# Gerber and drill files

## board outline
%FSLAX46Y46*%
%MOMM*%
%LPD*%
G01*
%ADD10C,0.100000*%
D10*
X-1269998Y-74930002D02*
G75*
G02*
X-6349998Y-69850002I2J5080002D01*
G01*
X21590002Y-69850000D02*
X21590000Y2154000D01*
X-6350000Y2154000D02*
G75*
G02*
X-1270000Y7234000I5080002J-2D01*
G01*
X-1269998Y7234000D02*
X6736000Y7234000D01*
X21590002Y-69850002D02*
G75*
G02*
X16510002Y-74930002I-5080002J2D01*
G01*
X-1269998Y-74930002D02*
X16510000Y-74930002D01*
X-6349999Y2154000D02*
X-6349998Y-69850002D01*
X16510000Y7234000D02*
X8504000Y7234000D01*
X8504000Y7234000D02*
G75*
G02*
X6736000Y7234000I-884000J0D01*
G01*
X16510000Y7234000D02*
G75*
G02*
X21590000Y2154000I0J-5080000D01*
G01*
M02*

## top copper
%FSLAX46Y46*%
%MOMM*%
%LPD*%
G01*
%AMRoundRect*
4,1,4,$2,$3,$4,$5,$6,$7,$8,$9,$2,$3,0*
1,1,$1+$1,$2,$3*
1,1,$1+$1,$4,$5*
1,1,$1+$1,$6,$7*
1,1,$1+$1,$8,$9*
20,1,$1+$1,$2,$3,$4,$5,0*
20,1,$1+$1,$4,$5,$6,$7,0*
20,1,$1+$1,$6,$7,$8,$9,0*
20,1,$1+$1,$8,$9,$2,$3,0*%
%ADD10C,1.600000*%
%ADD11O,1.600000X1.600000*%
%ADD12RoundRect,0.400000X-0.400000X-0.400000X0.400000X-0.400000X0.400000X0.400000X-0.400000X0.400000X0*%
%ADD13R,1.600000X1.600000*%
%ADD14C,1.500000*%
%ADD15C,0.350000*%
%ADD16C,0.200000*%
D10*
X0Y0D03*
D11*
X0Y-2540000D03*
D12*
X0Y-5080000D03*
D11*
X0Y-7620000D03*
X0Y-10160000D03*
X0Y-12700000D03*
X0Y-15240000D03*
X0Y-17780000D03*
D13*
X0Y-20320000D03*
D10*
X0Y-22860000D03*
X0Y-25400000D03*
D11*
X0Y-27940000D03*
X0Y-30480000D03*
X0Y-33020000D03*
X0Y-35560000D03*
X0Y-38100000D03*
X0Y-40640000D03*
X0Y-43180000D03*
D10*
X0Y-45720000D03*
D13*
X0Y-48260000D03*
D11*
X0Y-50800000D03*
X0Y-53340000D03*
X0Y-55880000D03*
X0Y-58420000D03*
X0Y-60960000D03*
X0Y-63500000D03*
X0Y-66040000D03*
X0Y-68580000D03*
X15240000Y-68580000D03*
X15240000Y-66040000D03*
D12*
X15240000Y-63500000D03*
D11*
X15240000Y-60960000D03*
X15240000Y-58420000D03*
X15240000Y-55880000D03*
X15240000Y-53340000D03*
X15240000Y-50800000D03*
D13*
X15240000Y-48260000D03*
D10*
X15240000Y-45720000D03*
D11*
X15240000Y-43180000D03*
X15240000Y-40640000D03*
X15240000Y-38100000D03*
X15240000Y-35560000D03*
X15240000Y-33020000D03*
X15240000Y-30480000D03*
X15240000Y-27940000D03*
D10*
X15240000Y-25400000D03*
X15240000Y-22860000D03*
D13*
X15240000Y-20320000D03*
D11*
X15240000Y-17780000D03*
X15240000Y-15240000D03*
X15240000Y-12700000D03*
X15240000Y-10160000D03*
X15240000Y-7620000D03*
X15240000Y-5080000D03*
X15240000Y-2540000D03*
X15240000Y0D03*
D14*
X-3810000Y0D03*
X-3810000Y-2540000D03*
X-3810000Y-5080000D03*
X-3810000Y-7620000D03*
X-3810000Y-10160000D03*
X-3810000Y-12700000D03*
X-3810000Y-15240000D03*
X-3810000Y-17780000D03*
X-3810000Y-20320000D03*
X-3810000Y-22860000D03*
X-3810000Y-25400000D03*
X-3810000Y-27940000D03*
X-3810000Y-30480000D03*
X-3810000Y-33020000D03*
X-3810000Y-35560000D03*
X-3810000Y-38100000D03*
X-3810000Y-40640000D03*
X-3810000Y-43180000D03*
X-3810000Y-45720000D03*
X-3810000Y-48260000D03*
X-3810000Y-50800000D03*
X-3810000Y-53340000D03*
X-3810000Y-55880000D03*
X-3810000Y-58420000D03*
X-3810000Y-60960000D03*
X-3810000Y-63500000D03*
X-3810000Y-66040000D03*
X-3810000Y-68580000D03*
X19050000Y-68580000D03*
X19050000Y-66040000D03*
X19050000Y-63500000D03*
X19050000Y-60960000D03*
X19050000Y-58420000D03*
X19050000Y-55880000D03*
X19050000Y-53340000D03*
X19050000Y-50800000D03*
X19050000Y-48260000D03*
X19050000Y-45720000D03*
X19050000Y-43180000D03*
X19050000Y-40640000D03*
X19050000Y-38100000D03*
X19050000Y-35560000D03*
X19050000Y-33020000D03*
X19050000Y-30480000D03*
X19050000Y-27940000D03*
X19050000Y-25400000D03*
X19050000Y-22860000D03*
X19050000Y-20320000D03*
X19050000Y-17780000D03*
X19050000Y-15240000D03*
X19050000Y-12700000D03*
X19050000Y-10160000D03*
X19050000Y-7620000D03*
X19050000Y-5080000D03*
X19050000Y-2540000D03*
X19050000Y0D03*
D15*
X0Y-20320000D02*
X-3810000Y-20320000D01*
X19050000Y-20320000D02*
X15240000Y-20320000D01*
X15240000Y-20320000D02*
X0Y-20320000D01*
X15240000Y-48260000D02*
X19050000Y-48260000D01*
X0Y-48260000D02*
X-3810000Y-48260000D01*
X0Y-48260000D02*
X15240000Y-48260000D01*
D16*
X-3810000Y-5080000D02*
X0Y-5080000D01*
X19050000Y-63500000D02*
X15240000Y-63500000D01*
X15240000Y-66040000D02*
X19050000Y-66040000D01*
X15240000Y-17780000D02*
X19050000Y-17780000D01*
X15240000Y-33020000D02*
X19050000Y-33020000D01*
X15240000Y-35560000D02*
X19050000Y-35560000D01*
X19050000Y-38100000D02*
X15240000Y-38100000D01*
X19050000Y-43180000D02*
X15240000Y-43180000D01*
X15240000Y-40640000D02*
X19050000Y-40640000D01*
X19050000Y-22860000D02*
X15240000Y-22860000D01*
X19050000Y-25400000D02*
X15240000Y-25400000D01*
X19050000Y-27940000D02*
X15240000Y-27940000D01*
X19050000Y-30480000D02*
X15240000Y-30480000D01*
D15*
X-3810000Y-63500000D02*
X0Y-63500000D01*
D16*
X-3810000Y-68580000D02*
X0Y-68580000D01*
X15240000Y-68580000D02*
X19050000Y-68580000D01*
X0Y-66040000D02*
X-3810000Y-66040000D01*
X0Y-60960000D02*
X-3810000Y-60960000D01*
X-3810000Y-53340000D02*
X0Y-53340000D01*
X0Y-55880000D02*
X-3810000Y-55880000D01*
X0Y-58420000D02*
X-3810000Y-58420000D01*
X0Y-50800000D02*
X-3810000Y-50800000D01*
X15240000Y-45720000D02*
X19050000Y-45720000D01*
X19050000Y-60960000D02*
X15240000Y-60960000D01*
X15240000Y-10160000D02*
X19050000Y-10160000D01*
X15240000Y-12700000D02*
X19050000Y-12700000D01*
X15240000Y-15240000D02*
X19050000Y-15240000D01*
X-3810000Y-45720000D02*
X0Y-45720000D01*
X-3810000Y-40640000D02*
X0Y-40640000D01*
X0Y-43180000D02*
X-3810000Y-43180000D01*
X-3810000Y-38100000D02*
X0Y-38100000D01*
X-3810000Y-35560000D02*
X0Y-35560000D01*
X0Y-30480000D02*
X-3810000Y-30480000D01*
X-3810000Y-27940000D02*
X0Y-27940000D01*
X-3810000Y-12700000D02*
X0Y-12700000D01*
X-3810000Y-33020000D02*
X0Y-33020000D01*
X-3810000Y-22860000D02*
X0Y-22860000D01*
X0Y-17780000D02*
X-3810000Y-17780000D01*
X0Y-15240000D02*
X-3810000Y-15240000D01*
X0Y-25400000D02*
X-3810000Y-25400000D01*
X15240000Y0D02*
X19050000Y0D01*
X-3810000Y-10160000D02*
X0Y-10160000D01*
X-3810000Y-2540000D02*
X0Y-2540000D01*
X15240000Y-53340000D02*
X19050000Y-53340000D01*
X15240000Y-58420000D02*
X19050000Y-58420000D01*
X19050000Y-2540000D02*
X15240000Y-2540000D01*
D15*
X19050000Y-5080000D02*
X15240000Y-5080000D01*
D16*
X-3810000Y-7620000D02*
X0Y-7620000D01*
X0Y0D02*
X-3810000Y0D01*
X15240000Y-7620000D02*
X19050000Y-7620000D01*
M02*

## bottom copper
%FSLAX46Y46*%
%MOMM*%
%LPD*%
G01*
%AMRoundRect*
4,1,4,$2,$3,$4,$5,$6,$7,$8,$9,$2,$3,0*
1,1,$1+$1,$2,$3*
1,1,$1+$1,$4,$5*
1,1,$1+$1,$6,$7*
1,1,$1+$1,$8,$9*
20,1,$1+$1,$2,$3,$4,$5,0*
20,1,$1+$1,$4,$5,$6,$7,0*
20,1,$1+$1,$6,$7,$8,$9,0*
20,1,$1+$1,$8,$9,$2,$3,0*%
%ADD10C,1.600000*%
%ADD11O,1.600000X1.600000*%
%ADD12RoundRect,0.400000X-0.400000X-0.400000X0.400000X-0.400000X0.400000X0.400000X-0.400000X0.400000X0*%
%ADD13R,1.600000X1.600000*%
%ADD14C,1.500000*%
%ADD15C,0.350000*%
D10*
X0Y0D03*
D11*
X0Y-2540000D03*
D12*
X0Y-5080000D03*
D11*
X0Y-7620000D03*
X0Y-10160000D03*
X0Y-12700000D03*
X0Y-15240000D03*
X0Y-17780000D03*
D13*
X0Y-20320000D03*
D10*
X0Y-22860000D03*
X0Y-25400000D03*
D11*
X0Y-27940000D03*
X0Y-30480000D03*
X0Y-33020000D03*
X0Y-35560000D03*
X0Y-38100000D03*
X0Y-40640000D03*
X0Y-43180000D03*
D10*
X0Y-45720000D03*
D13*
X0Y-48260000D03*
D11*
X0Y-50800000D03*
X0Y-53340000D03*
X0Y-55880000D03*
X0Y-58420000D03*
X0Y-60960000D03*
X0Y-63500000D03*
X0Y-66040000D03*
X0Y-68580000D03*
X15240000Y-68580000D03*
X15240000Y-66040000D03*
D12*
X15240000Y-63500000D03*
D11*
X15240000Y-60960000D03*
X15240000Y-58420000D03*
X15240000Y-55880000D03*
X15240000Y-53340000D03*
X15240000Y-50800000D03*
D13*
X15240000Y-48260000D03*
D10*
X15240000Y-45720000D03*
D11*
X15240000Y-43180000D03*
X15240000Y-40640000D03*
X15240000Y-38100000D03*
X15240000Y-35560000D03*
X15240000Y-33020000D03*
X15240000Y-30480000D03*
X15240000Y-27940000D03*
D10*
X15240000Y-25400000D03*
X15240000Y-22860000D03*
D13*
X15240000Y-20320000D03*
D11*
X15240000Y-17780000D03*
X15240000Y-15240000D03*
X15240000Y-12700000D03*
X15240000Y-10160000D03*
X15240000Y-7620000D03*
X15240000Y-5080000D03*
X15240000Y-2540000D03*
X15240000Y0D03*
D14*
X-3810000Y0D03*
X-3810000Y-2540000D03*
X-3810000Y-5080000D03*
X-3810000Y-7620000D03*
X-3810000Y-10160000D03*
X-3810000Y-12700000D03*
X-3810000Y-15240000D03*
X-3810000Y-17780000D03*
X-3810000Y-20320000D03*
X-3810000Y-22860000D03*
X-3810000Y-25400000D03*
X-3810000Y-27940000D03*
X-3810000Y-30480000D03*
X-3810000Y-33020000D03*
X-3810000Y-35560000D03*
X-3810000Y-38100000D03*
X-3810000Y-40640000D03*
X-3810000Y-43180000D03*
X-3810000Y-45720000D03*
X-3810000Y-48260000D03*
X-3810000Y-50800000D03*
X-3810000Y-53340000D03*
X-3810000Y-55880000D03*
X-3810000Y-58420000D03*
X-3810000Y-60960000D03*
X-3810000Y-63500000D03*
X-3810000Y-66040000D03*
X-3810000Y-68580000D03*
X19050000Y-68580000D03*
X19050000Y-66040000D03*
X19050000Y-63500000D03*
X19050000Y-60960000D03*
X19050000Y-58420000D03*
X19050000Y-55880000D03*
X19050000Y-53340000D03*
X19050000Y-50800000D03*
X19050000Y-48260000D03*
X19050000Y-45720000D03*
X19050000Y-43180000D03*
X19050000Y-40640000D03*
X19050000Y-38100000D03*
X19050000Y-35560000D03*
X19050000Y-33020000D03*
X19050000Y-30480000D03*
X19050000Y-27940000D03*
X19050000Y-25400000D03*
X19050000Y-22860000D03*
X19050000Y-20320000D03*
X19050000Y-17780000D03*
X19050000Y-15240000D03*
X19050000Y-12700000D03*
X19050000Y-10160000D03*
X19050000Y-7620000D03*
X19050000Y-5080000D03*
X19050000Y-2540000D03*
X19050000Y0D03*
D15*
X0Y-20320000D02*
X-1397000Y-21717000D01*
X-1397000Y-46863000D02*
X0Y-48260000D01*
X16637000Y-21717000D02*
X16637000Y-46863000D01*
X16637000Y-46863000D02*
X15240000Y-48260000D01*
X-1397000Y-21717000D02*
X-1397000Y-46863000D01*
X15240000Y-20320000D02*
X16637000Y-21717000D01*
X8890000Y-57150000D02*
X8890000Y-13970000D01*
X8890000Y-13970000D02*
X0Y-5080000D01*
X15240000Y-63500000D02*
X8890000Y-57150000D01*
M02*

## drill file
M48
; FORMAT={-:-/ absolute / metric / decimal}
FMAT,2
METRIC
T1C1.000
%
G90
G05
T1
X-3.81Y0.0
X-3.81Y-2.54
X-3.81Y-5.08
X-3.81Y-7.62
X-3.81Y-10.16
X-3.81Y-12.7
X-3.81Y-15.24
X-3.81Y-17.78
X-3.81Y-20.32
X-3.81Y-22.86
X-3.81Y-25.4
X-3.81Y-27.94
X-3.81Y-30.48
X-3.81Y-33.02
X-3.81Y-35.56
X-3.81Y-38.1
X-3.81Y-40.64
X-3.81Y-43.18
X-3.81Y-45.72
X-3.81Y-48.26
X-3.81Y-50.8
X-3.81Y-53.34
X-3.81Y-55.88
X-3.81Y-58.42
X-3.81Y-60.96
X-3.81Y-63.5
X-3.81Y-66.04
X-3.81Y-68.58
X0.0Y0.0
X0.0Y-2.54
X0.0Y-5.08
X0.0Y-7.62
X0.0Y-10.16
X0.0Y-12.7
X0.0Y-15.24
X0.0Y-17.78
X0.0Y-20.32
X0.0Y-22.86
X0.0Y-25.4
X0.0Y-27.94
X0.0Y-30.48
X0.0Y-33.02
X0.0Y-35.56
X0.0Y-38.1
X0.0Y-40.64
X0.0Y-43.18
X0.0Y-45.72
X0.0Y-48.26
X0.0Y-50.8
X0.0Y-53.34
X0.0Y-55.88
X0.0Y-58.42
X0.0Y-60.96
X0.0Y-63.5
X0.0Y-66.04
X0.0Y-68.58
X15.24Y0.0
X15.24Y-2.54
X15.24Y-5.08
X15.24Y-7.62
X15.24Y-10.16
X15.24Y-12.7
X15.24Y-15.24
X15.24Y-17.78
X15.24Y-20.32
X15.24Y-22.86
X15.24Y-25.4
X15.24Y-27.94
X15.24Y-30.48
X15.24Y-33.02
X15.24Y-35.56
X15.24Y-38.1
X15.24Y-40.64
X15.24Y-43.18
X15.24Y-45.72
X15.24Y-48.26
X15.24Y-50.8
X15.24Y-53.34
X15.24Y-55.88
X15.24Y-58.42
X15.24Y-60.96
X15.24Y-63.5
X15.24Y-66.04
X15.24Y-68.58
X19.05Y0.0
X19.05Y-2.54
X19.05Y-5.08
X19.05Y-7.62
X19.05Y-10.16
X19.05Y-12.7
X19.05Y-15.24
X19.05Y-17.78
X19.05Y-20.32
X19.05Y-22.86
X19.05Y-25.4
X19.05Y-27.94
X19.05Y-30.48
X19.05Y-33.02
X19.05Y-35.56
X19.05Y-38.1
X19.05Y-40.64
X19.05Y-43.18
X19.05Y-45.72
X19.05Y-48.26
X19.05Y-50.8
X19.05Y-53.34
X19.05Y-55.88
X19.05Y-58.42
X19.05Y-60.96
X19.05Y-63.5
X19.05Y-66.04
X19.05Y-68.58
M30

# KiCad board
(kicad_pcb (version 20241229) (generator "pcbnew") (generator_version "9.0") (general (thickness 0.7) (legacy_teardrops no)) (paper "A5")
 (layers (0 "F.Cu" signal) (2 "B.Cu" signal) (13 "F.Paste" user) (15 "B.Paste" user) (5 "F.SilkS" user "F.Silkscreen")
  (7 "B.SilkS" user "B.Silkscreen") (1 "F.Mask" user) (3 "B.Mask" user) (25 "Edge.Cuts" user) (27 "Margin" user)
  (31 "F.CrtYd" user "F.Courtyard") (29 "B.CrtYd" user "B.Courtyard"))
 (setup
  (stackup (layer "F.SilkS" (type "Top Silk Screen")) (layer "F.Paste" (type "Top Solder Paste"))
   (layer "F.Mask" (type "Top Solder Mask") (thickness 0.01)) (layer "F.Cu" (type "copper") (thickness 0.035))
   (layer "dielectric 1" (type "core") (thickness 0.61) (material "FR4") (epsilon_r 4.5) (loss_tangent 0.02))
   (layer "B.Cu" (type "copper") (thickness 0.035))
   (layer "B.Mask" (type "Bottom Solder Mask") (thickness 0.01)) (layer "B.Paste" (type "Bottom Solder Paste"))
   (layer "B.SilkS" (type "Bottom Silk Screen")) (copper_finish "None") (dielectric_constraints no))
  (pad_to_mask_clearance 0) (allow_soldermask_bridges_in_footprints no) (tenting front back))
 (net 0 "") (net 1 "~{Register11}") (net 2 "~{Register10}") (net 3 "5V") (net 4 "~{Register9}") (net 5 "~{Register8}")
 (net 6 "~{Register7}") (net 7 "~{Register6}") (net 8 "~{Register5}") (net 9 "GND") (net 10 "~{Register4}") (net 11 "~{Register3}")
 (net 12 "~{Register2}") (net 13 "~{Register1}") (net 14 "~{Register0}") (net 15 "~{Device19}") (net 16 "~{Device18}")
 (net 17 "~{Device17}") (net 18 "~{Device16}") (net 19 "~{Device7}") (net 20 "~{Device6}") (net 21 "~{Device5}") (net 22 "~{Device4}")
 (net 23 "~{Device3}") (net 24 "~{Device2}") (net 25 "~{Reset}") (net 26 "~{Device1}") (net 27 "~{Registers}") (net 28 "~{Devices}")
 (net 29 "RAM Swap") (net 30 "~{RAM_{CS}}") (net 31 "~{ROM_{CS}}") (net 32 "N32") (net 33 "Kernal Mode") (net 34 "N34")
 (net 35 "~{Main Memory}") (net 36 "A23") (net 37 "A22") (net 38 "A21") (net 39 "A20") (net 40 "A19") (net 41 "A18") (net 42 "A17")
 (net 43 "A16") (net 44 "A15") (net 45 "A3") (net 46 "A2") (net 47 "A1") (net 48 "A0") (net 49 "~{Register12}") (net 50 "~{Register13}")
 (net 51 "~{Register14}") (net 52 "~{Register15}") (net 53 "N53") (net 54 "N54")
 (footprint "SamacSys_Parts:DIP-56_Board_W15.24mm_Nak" (layer "F.Cu") (at 0 0)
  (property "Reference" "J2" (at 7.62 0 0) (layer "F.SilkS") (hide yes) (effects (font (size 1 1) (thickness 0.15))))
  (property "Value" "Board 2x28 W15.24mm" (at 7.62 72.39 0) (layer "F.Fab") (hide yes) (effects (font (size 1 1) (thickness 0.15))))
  (pad "1" thru_hole circle (at 0 0) (size 1.6 1.6) (drill 1) (layers "*.Cu" "*.Mask") (remove_unused_layers no) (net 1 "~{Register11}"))
  (pad "2" thru_hole oval (at 0 2.54) (size 1.6 1.6) (drill 1) (layers "*.Cu" "*.Mask") (remove_unused_layers no) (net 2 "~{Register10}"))
  (pad "3" thru_hole roundrect (at 0 5.08) (size 1.6 1.6) (drill 1) (layers "*.Cu" "*.Mask") (remove_unused_layers no)
   (roundrect_rratio 0.25) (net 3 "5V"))
  (pad "4" thru_hole oval (at 0 7.62) (size 1.6 1.6) (drill 1) (layers "*.Cu" "*.Mask") (remove_unused_layers no) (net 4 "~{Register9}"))
  (pad "5" thru_hole oval (at 0 10.16) (size 1.6 1.6) (drill 1) (layers "*.Cu" "*.Mask") (remove_unused_layers no) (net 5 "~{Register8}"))
  (pad "6" thru_hole oval (at 0 12.7) (size 1.6 1.6) (drill 1) (layers "*.Cu" "*.Mask") (remove_unused_layers no) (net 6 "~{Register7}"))
  (pad "7" thru_hole oval (at 0 15.24) (size 1.6 1.6) (drill 1) (layers "*.Cu" "*.Mask") (remove_unused_layers no) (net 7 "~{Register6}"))
  (pad "8" thru_hole oval (at 0 17.78) (size 1.6 1.6) (drill 1) (layers "*.Cu" "*.Mask") (remove_unused_layers no) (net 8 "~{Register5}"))
  (pad "9" thru_hole rect (at 0 20.32) (size 1.6 1.6) (drill 1) (layers "*.Cu" "*.Mask") (remove_unused_layers no) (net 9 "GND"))
  (pad "10" thru_hole circle (at 0 22.86) (size 1.6 1.6) (drill 1) (layers "*.Cu" "*.Mask") (remove_unused_layers no)
   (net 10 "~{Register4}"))
  (pad "11" thru_hole circle (at 0 25.4) (size 1.6 1.6) (drill 1) (layers "*.Cu" "*.Mask") (remove_unused_layers no) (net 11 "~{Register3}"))
  (pad "12" thru_hole oval (at 0 27.94) (size 1.6 1.6) (drill 1) (layers "*.Cu" "*.Mask") (remove_unused_layers no) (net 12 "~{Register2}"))
  (pad "13" thru_hole oval (at 0 30.48) (size 1.6 1.6) (drill 1) (layers "*.Cu" "*.Mask") (remove_unused_layers no) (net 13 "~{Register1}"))
  (pad "14" thru_hole oval (at 0 33.02) (size 1.6 1.6) (drill 1) (layers "*.Cu" "*.Mask") (remove_unused_layers no) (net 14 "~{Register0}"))
  (pad "15" thru_hole oval (at 0 35.56) (size 1.6 1.6) (drill 1) (layers "*.Cu" "*.Mask") (remove_unused_layers no) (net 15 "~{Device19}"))
  (pad "16" thru_hole oval (at 0 38.1) (size 1.6 1.6) (drill 1) (layers "*.Cu" "*.Mask") (remove_unused_layers no) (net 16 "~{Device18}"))
  (pad "17" thru_hole oval (at 0 40.64) (size 1.6 1.6) (drill 1) (layers "*.Cu" "*.Mask") (remove_unused_layers no) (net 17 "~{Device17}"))
  (pad "18" thru_hole oval (at 0 43.18) (size 1.6 1.6) (drill 1) (layers "*.Cu" "*.Mask") (remove_unused_layers no) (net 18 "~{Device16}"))
  (pad "19" thru_hole circle (at 0 45.72) (size 1.6 1.6) (drill 1) (layers "*.Cu" "*.Mask") (remove_unused_layers no) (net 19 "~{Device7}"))
  (pad "20" thru_hole rect (at 0 48.26) (size 1.6 1.6) (drill 1) (layers "*.Cu" "*.Mask") (remove_unused_layers no) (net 9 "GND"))
  (pad "21" thru_hole oval (at 0 50.8) (size 1.6 1.6) (drill 1) (layers "*.Cu" "*.Mask") (remove_unused_layers no) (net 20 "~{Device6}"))
  (pad "22" thru_hole oval (at 0 53.34) (size 1.6 1.6) (drill 1) (layers "*.Cu" "*.Mask") (remove_unused_layers no) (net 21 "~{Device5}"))
  (pad "23" thru_hole oval (at 0 55.88) (size 1.6 1.6) (drill 1) (layers "*.Cu" "*.Mask") (remove_unused_layers no) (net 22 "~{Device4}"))
  (pad "24" thru_hole oval (at 0 58.42) (size 1.6 1.6) (drill 1) (layers "*.Cu" "*.Mask") (remove_unused_layers no) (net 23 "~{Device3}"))
  (pad "25" thru_hole oval (at 0 60.96) (size 1.6 1.6) (drill 1) (layers "*.Cu" "*.Mask") (remove_unused_layers no) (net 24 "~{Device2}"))
  (pad "26" thru_hole oval (at 0 63.5) (size 1.6 1.6) (drill 1) (layers "*.Cu" "*.Mask") (remove_unused_layers no) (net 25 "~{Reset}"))
  (pad "27" thru_hole oval (at 0 66.04) (size 1.6 1.6) (drill 1) (layers "*.Cu" "*.Mask") (remove_unused_layers no) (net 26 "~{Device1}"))
  (pad "28" thru_hole oval (at 0 68.58) (size 1.6 1.6) (drill 1) (layers "*.Cu" "*.Mask") (remove_unused_layers no) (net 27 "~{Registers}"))
  (pad "29" thru_hole oval (at 15.24 68.58) (size 1.6 1.6) (drill 1) (layers "*.Cu" "*.Mask") (remove_unused_layers no)
   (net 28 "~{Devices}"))
  (pad "30" thru_hole oval (at 15.24 66.04) (size 1.6 1.6) (drill 1) (layers "*.Cu" "*.Mask") (remove_unused_layers no) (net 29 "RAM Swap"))
  (pad "31" thru_hole roundrect (at 15.24 63.5) (size 1.6 1.6) (drill 1) (layers "*.Cu" "*.Mask") (remove_unused_layers no)
   (roundrect_rratio 0.25) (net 3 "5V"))
  (pad "32" thru_hole oval (at 15.24 60.96) (size 1.6 1.6) (drill 1) (layers "*.Cu" "*.Mask") (remove_unused_layers no)
   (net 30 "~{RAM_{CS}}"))
  (pad "33" thru_hole oval (at 15.24 58.42) (size 1.6 1.6) (drill 1) (layers "*.Cu" "*.Mask") (remove_unused_layers no)
   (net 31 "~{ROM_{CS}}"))
  (pad "34" thru_hole oval (at 15.24 55.88) (size 1.6 1.6) (drill 1) (layers "*.Cu" "*.Mask") (remove_unused_layers no) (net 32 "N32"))
  (pad "35" thru_hole oval (at 15.24 53.34) (size 1.6 1.6) (drill 1) (layers "*.Cu" "*.Mask") (remove_unused_layers no)
   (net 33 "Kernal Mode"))
  (pad "36" thru_hole oval (at 15.24 50.8) (size 1.6 1.6) (drill 1) (layers "*.Cu" "*.Mask") (remove_unused_layers no) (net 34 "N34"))
  (pad "37" thru_hole rect (at 15.24 48.26) (size 1.6 1.6) (drill 1) (layers "*.Cu" "*.Mask") (remove_unused_layers no) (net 9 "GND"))
  (pad "38" thru_hole circle (at 15.24 45.72) (size 1.6 1.6) (drill 1) (layers "*.Cu" "*.Mask") (remove_unused_layers no)
   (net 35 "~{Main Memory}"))
  (pad "39" thru_hole oval (at 15.24 43.18) (size 1.6 1.6) (drill 1) (layers "*.Cu" "*.Mask") (remove_unused_layers no) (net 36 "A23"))
  (pad "40" thru_hole oval (at 15.24 40.64) (size 1.6 1.6) (drill 1) (layers "*.Cu" "*.Mask") (remove_unused_layers no) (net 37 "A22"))
  (pad "41" thru_hole oval (at 15.24 38.1) (size 1.6 1.6) (drill 1) (layers "*.Cu" "*.Mask") (remove_unused_layers no) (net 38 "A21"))
  (pad "42" thru_hole oval (at 15.24 35.56) (size 1.6 1.6) (drill 1) (layers "*.Cu" "*.Mask") (remove_unused_layers no) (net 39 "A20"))
  (pad "43" thru_hole oval (at 15.24 33.02) (size 1.6 1.6) (drill 1) (layers "*.Cu" "*.Mask") (remove_unused_layers no) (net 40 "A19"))
  (pad "44" thru_hole oval (at 15.24 30.48) (size 1.6 1.6) (drill 1) (layers "*.Cu" "*.Mask") (remove_unused_layers no) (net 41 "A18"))
  (pad "45" thru_hole oval (at 15.24 27.94) (size 1.6 1.6) (drill 1) (layers "*.Cu" "*.Mask") (remove_unused_layers no) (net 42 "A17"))
  (pad "46" thru_hole circle (at 15.24 25.4) (size 1.6 1.6) (drill 1) (layers "*.Cu" "*.Mask") (remove_unused_layers no) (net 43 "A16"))
  (pad "47" thru_hole circle (at 15.24 22.86) (size 1.6 1.6) (drill 1) (layers "*.Cu" "*.Mask") (remove_unused_layers no) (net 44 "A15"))
  (pad "48" thru_hole rect (at 15.24 20.32) (size 1.6 1.6) (drill 1) (layers "*.Cu" "*.Mask") (remove_unused_layers no) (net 9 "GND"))
  (pad "49" thru_hole oval (at 15.24 17.78) (size 1.6 1.6) (drill 1) (layers "*.Cu" "*.Mask") (remove_unused_layers no) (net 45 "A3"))
  (pad "50" thru_hole oval (at 15.24 15.24) (size 1.6 1.6) (drill 1) (layers "*.Cu" "*.Mask") (remove_unused_layers no) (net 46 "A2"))
  (pad "51" thru_hole oval (at 15.24 12.7) (size 1.6 1.6) (drill 1) (layers "*.Cu" "*.Mask") (remove_unused_layers no) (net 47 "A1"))
  (pad "52" thru_hole oval (at 15.24 10.16) (size 1.6 1.6) (drill 1) (layers "*.Cu" "*.Mask") (remove_unused_layers no) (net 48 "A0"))
  (pad "53" thru_hole oval (at 15.24 7.62) (size 1.6 1.6) (drill 1) (layers "*.Cu" "*.Mask") (remove_unused_layers no)
   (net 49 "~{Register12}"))
  (pad "54" thru_hole oval (at 15.24 5.08) (size 1.6 1.6) (drill 1) (layers "*.Cu" "*.Mask") (remove_unused_layers no)
   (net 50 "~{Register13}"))
  (pad "55" thru_hole oval (at 15.24 2.54) (size 1.6 1.6) (drill 1) (layers "*.Cu" "*.Mask") (remove_unused_layers no)
   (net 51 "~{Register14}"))
  (pad "56" thru_hole oval (at 15.24 0) (size 1.6 1.6) (drill 1) (layers "*.Cu" "*.Mask") (remove_unused_layers no) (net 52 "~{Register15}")))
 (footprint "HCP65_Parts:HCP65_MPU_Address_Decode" (layer "F.Cu") (at -3.81 0)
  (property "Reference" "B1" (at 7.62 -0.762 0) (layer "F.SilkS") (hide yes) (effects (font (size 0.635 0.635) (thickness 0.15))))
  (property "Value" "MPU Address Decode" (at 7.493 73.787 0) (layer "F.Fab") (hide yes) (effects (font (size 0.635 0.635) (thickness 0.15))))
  (pad "1" thru_hole circle (at 0 0) (size 1.5 1.5) (drill 1) (layers "*.Cu" "*.Mask") (remove_unused_layers no) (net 1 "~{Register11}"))
  (pad "2" thru_hole circle (at 0 2.54) (size 1.5 1.5) (drill 1) (layers "*.Cu" "*.Mask") (remove_unused_layers no) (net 2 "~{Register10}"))
  (pad "3" thru_hole circle (at 0 5.08) (size 1.5 1.5) (drill 1) (layers "*.Cu" "*.Mask") (remove_unused_layers no) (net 3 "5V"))
  (pad "4" thru_hole circle (at 0 7.62) (size 1.5 1.5) (drill 1) (layers "*.Cu" "*.Mask") (remove_unused_layers no) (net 4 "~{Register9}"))
  (pad "5" thru_hole circle (at 0 10.16) (size 1.5 1.5) (drill 1) (layers "*.Cu" "*.Mask") (remove_unused_layers no) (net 5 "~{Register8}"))
  (pad "6" thru_hole circle (at 0 12.7) (size 1.5 1.5) (drill 1) (layers "*.Cu" "*.Mask") (remove_unused_layers no) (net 6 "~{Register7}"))
  (pad "7" thru_hole circle (at 0 15.24) (size 1.5 1.5) (drill 1) (layers "*.Cu" "*.Mask") (remove_unused_layers no) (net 7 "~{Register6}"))
  (pad "8" thru_hole circle (at 0 17.78) (size 1.5 1.5) (drill 1) (layers "*.Cu" "*.Mask") (remove_unused_layers no) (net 8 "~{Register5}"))
  (pad "9" thru_hole circle (at 0 20.32) (size 1.5 1.5) (drill 1) (layers "*.Cu" "*.Mask") (remove_unused_layers no) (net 9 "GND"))
  (pad "10" thru_hole circle (at 0 22.86) (size 1.5 1.5) (drill 1) (layers "*.Cu" "*.Mask") (remove_unused_layers no)
   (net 10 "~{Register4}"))
  (pad "11" thru_hole circle (at 0 25.4) (size 1.5 1.5) (drill 1) (layers "*.Cu" "*.Mask") (remove_unused_layers no) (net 11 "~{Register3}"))
  (pad "12" thru_hole circle (at 0 27.94) (size 1.5 1.5) (drill 1) (layers "*.Cu" "*.Mask") (remove_unused_layers no)
   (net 12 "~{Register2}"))
  (pad "13" thru_hole circle (at 0 30.48) (size 1.5 1.5) (drill 1) (layers "*.Cu" "*.Mask") (remove_unused_layers no)
   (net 13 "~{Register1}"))
  (pad "14" thru_hole circle (at 0 33.02) (size 1.5 1.5) (drill 1) (layers "*.Cu" "*.Mask") (remove_unused_layers no)
   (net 14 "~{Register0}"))
  (pad "15" thru_hole circle (at 0 35.56) (size 1.5 1.5) (drill 1) (layers "*.Cu" "*.Mask") (remove_unused_layers no) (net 15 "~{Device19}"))
  (pad "16" thru_hole circle (at 0 38.1) (size 1.5 1.5) (drill 1) (layers "*.Cu" "*.Mask") (remove_unused_layers no) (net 16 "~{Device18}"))
  (pad "17" thru_hole circle (at 0 40.64) (size 1.5 1.5) (drill 1) (layers "*.Cu" "*.Mask") (remove_unused_layers no) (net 17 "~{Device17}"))
  (pad "18" thru_hole circle (at 0 43.18) (size 1.5 1.5) (drill 1) (layers "*.Cu" "*.Mask") (remove_unused_layers no) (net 18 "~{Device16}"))
  (pad "19" thru_hole circle (at 0 45.72) (size 1.5 1.5) (drill 1) (layers "*.Cu" "*.Mask") (remove_unused_layers no) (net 19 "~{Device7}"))
  (pad "20" thru_hole circle (at 0 48.26) (size 1.5 1.5) (drill 1) (layers "*.Cu" "*.Mask") (remove_unused_layers no) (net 9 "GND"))
  (pad "21" thru_hole circle (at 0 50.8) (size 1.5 1.5) (drill 1) (layers "*.Cu" "*.Mask") (remove_unused_layers no) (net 20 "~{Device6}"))
  (pad "22" thru_hole circle (at 0 53.34) (size 1.5 1.5) (drill 1) (layers "*.Cu" "*.Mask") (remove_unused_layers no) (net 21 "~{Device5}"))
  (pad "23" thru_hole circle (at 0 55.88) (size 1.5 1.5) (drill 1) (layers "*.Cu" "*.Mask") (remove_unused_layers no) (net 22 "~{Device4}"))
  (pad "24" thru_hole circle (at 0 58.42) (size 1.5 1.5) (drill 1) (layers "*.Cu" "*.Mask") (remove_unused_layers no) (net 23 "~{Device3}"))
  (pad "25" thru_hole circle (at 0 60.96) (size 1.5 1.5) (drill 1) (layers "*.Cu" "*.Mask") (remove_unused_layers no) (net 24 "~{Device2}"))
  (pad "26" thru_hole circle (at 0 63.5) (size 1.5 1.5) (drill 1) (layers "*.Cu" "*.Mask") (remove_unused_layers no) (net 25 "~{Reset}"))
  (pad "27" thru_hole circle (at 0 66.04) (size 1.5 1.5) (drill 1) (layers "*.Cu" "*.Mask") (remove_unused_layers no) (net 26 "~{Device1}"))
  (pad "28" thru_hole circle (at 0 68.58) (size 1.5 1.5) (drill 1) (layers "*.Cu" "*.Mask") (remove_unused_layers no)
   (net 27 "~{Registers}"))
  (pad "29" thru_hole circle (at 22.86 68.58) (size 1.5 1.5) (drill 1) (layers "*.Cu" "*.Mask") (remove_unused_layers no)
   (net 28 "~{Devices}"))
  (pad "30" thru_hole circle (at 22.86 66.04) (size 1.5 1.5) (drill 1) (layers "*.Cu" "*.Mask") (remove_unused_layers no)
   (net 29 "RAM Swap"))
  (pad "31" thru_hole circle (at 22.86 63.5) (size 1.5 1.5) (drill 1) (layers "*.Cu" "*.Mask") (remove_unused_layers no) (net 3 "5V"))
  (pad "32" thru_hole circle (at 22.86 60.96) (size 1.5 1.5) (drill 1) (layers "*.Cu" "*.Mask") (remove_unused_layers no)
   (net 30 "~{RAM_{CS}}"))
  (pad "33" thru_hole circle (at 22.86 58.42) (size 1.5 1.5) (drill 1) (layers "*.Cu" "*.Mask") (remove_unused_layers no)
   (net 31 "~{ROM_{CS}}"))
  (pad "34" thru_hole circle (at 22.86 55.88) (size 1.5 1.5) (drill 1) (layers "*.Cu" "*.Mask") (remove_unused_layers no) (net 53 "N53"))
  (pad "35" thru_hole circle (at 22.86 53.34) (size 1.5 1.5) (drill 1) (layers "*.Cu" "*.Mask") (remove_unused_layers no)
   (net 33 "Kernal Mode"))
  (pad "36" thru_hole circle (at 22.86 50.8) (size 1.5 1.5) (drill 1) (layers "*.Cu" "*.Mask") (remove_unused_layers no) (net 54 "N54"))
  (pad "37" thru_hole circle (at 22.86 48.26) (size 1.5 1.5) (drill 1) (layers "*.Cu" "*.Mask") (remove_unused_layers no) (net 9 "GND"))
  (pad "38" thru_hole circle (at 22.86 45.72) (size 1.5 1.5) (drill 1) (layers "*.Cu" "*.Mask") (remove_unused_layers no)
   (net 35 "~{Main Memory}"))
  (pad "39" thru_hole circle (at 22.86 43.18) (size 1.5 1.5) (drill 1) (layers "*.Cu" "*.Mask") (remove_unused_layers no) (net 36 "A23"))
  (pad "40" thru_hole circle (at 22.86 40.64) (size 1.5 1.5) (drill 1) (layers "*.Cu" "*.Mask") (remove_unused_layers no) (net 37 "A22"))
  (pad "41" thru_hole circle (at 22.86 38.1) (size 1.5 1.5) (drill 1) (layers "*.Cu" "*.Mask") (remove_unused_layers no) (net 38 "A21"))
  (pad "42" thru_hole circle (at 22.86 35.56) (size 1.5 1.5) (drill 1) (layers "*.Cu" "*.Mask") (remove_unused_layers no) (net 39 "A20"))
  (pad "43" thru_hole circle (at 22.86 33.02) (size 1.5 1.5) (drill 1) (layers "*.Cu" "*.Mask") (remove_unused_layers no) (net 40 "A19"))
  (pad "44" thru_hole circle (at 22.86 30.48) (size 1.5 1.5) (drill 1) (layers "*.Cu" "*.Mask") (remove_unused_layers no) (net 41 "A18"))
  (pad "45" thru_hole circle (at 22.86 27.94) (size 1.5 1.5) (drill 1) (layers "*.Cu" "*.Mask") (remove_unused_layers no) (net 42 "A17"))
  (pad "46" thru_hole circle (at 22.86 25.4) (size 1.5 1.5) (drill 1) (layers "*.Cu" "*.Mask") (remove_unused_layers no) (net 43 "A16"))
  (pad "47" thru_hole circle (at 22.86 22.86) (size 1.5 1.5) (drill 1) (layers "*.Cu" "*.Mask") (remove_unused_layers no) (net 44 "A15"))
  (pad "48" thru_hole circle (at 22.86 20.32) (size 1.5 1.5) (drill 1) (layers "*.Cu" "*.Mask") (remove_unused_layers no) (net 9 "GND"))
  (pad "49" thru_hole circle (at 22.86 17.78) (size 1.5 1.5) (drill 1) (layers "*.Cu" "*.Mask") (remove_unused_layers no) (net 45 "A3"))
  (pad "50" thru_hole circle (at 22.86 15.24) (size 1.5 1.5) (drill 1) (layers "*.Cu" "*.Mask") (remove_unused_layers no) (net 46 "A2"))
  (pad "51" thru_hole circle (at 22.86 12.7) (size 1.5 1.5) (drill 1) (layers "*.Cu" "*.Mask") (remove_unused_layers no) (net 47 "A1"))
  (pad "52" thru_hole circle (at 22.86 10.16) (size 1.5 1.5) (drill 1) (layers "*.Cu" "*.Mask") (remove_unused_layers no) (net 48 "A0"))
  (pad "53" thru_hole circle (at 22.86 7.62) (size 1.5 1.5) (drill 1) (layers "*.Cu" "*.Mask") (remove_unused_layers no)
   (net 49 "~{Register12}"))
  (pad "54" thru_hole circle (at 22.86 5.08) (size 1.5 1.5) (drill 1) (layers "*.Cu" "*.Mask") (remove_unused_layers no)
   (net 50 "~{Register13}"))
  (pad "55" thru_hole circle (at 22.86 2.54) (size 1.5 1.5) (drill 1) (layers "*.Cu" "*.Mask") (remove_unused_layers no)
   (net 51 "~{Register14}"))
  (pad "56" thru_hole circle (at 22.86 0) (size 1.5 1.5) (drill 1) (layers "*.Cu" "*.Mask") (remove_unused_layers no)
   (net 52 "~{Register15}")))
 (gr_arc (start -1.269998 74.930002) (mid -4.8621 73.442104) (end -6.349998 69.850002) (stroke (width 0.1) (type default))
  (layer "Edge.Cuts"))
 (gr_line (start 21.590002 69.85) (end 21.59 -2.154) (stroke (width 0.1) (type default)) (layer "Edge.Cuts"))
 (gr_arc (start -6.35 -2.154) (mid -4.862102 -5.746102) (end -1.27 -7.234) (stroke (width 0.1) (type default)) (layer "Edge.Cuts"))
 (gr_line (start -1.269998 -7.234) (end 6.736 -7.234) (stroke (width 0.1) (type default)) (layer "Edge.Cuts"))
 (gr_arc (start 21.590002 69.850002) (mid 20.102104 73.442104) (end 16.510002 74.930002) (stroke (width 0.1) (type default))
  (layer "Edge.Cuts"))
 (gr_line (start -1.269998 74.930002) (end 16.51 74.930002) (stroke (width 0.1) (type solid)) (layer "Edge.Cuts"))
 (gr_line (start -6.349999 -2.154) (end -6.349998 69.850002) (stroke (width 0.1) (type default)) (layer "Edge.Cuts"))
 (gr_line (start 16.51 -7.234) (end 8.504 -7.234) (stroke (width 0.1) (type solid)) (layer "Edge.Cuts"))
 (gr_arc (start 8.504 -7.234) (mid 7.62 -6.35) (end 6.736 -7.234) (stroke (width 0.1) (type solid)) (layer "Edge.Cuts"))
 (gr_arc (start 16.51 -7.234) (mid 20.102102 -5.746102) (end 21.59 -2.154) (stroke (width 0.1) (type default)) (layer "Edge.Cuts"))
 (segment (start 0 20.32) (end -3.81 20.32) (width 0.35) (layer "F.Cu") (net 9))
 (segment (start 19.05 20.32) (end 15.24 20.32) (width 0.35) (layer "F.Cu") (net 9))
 (segment (start 15.24 20.32) (end 0 20.32) (width 0.35) (layer "F.Cu") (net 9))
 (segment (start 15.24 48.26) (end 19.05 48.26) (width 0.35) (layer "F.Cu") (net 9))
 (segment (start 0 48.26) (end -3.81 48.26) (width 0.35) (layer "F.Cu") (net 9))
 (segment (start 0 48.26) (end 15.24 48.26) (width 0.35) (layer "F.Cu") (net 9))
 (segment (start 0 20.32) (end -1.397 21.717) (width 0.35) (layer "B.Cu") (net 9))
 (segment (start -1.397 46.863) (end 0 48.26) (width 0.35) (layer "B.Cu") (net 9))
 (segment (start 16.637 21.717) (end 16.637 46.863) (width 0.35) (layer "B.Cu") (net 9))
 (segment (start 16.637 46.863) (end 15.24 48.26) (width 0.35) (layer "B.Cu") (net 9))
 (segment (start -1.397 21.717) (end -1.397 46.863) (width 0.35) (layer "B.Cu") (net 9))
 (segment (start 15.24 20.32) (end 16.637 21.717) (width 0.35) (layer "B.Cu") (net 9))
 (segment (start -3.81 5.08) (end 0 5.08) (width 0.2) (layer "F.Cu") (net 3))
 (segment (start 19.05 63.5) (end 15.24 63.5) (width 0.2) (layer "F.Cu") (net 3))
 (segment (start 8.89 57.15) (end 8.89 13.97) (width 0.35) (layer "B.Cu") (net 3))
 (segment (start 8.89 13.97) (end 0 5.08) (width 0.35) (layer "B.Cu") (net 3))
 (segment (start 15.24 63.5) (end 8.89 57.15) (width 0.35) (layer "B.Cu") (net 3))
 (segment (start 15.24 66.04) (end 19.05 66.04) (width 0.2) (layer "F.Cu") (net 29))
 (segment (start 15.24 17.78) (end 19.05 17.78) (width 0.2) (layer "F.Cu") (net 45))
 (segment (start 15.24 33.02) (end 19.05 33.02) (width 0.2) (layer "F.Cu") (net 40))
 (segment (start 15.24 35.56) (end 19.05 35.56) (width 0.2) (layer "F.Cu") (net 39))
 (segment (start 19.05 38.1) (end 15.24 38.1) (width 0.2) (layer "F.Cu") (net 38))
 (segment (start 19.05 43.18) (end 15.24 43.18) (width 0.2) (layer "F.Cu") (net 36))
 (segment (start 15.24 40.64) (end 19.05 40.64) (width 0.2) (layer "F.Cu") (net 37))
 (segment (start 19.05 22.86) (end 15.24 22.86) (width 0.2) (layer "F.Cu") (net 44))
 (segment (start 19.05 25.4) (end 15.24 25.4) (width 0.2) (layer "F.Cu") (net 43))
 (segment (start 19.05 27.94) (end 15.24 27.94) (width 0.2) (layer "F.Cu") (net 42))
 (segment (start 19.05 30.48) (end 15.24 30.48) (width 0.2) (layer "F.Cu") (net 41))
 (segment (start -3.81 63.5) (end 0 63.5) (width 0.35) (layer "F.Cu") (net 25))
 (segment (start -3.81 68.58) (end 0 68.58) (width 0.2) (layer "F.Cu") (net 27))
 (segment (start 15.24 68.58) (end 19.05 68.58) (width 0.2) (layer "F.Cu") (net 28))
 (segment (start 0 66.04) (end -3.81 66.04) (width 0.2) (layer "F.Cu") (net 26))
 (segment (start 0 60.96) (end -3.81 60.96) (width 0.2) (layer "F.Cu") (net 24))
 (segment (start -3.81 53.34) (end 0 53.34) (width 0.2) (layer "F.Cu") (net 21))
 (segment (start 0 55.88) (end -3.81 55.88) (width 0.2) (layer "F.Cu") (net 22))
 (segment (start 0 58.42) (end -3.81 58.42) (width 0.2) (layer "F.Cu") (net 23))
 (segment (start 0 50.8) (end -3.81 50.8) (width 0.2) (layer "F.Cu") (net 20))
 (segment (start 15.24 45.72) (end 19.05 45.72) (width 0.2) (layer "F.Cu") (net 35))
 (segment (start 19.05 60.96) (end 15.24 60.96) (width 0.2) (layer "F.Cu") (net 30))
 (segment (start 15.24 10.16) (end 19.05 10.16) (width 0.2) (layer "F.Cu") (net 48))
 (segment (start 15.24 12.7) (end 19.05 12.7) (width 0.2) (layer "F.Cu") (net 47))
 (segment (start 15.24 15.24) (end 19.05 15.24) (width 0.2) (layer "F.Cu") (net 46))
 (segment (start -3.81 45.72) (end 0 45.72) (width 0.2) (layer "F.Cu") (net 19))
 (segment (start -3.81 40.64) (end 0 40.64) (width 0.2) (layer "F.Cu") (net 17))
 (segment (start 0 43.18) (end -3.81 43.18) (width 0.2) (layer "F.Cu") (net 18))
 (segment (start -3.81 38.1) (end 0 38.1) (width 0.2) (layer "F.Cu") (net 16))
 (segment (start -3.81 35.56) (end 0 35.56) (width 0.2) (layer "F.Cu") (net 15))
 (segment (start 0 30.48) (end -3.81 30.48) (width 0.2) (layer "F.Cu") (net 13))
 (segment (start -3.81 27.94) (end 0 27.94) (width 0.2) (layer "F.Cu") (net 12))
 (segment (start -3.81 12.7) (end 0 12.7) (width 0.2) (layer "F.Cu") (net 6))
 (segment (start -3.81 33.02) (end 0 33.02) (width 0.2) (layer "F.Cu") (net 14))
 (segment (start -3.81 22.86) (end 0 22.86) (width 0.2) (layer "F.Cu") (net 10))
 (segment (start 0 17.78) (end -3.81 17.78) (width 0.2) (layer "F.Cu") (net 8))
 (segment (start 0 15.24) (end -3.81 15.24) (width 0.2) (layer "F.Cu") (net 7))
 (segment (start 0 25.4) (end -3.81 25.4) (width 0.2) (layer "F.Cu") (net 11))
 (segment (start 15.24 0) (end 19.05 0) (width 0.2) (layer "F.Cu") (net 52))
 (segment (start -3.81 10.16) (end 0 10.16) (width 0.2) (layer "F.Cu") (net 5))
 (segment (start -3.81 2.54) (end 0 2.54) (width 0.2) (layer "F.Cu") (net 2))
 (segment (start 15.24 53.34) (end 19.05 53.34) (width 0.2) (layer "F.Cu") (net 33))
 (segment (start 15.24 58.42) (end 19.05 58.42) (width 0.2) (layer "F.Cu") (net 31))
 (segment (start 19.05 2.54) (end 15.24 2.54) (width 0.2) (layer "F.Cu") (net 51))
 (segment (start 19.05 5.08) (end 15.24 5.08) (width 0.35) (layer "F.Cu") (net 50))
 (segment (start -3.81 7.62) (end 0 7.62) (width 0.2) (layer "F.Cu") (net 4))
 (segment (start 0 0) (end -3.81 0) (width 0.2) (layer "F.Cu") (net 1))
 (segment (start 15.24 7.62) (end 19.05 7.62) (width 0.2) (layer "F.Cu") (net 49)))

